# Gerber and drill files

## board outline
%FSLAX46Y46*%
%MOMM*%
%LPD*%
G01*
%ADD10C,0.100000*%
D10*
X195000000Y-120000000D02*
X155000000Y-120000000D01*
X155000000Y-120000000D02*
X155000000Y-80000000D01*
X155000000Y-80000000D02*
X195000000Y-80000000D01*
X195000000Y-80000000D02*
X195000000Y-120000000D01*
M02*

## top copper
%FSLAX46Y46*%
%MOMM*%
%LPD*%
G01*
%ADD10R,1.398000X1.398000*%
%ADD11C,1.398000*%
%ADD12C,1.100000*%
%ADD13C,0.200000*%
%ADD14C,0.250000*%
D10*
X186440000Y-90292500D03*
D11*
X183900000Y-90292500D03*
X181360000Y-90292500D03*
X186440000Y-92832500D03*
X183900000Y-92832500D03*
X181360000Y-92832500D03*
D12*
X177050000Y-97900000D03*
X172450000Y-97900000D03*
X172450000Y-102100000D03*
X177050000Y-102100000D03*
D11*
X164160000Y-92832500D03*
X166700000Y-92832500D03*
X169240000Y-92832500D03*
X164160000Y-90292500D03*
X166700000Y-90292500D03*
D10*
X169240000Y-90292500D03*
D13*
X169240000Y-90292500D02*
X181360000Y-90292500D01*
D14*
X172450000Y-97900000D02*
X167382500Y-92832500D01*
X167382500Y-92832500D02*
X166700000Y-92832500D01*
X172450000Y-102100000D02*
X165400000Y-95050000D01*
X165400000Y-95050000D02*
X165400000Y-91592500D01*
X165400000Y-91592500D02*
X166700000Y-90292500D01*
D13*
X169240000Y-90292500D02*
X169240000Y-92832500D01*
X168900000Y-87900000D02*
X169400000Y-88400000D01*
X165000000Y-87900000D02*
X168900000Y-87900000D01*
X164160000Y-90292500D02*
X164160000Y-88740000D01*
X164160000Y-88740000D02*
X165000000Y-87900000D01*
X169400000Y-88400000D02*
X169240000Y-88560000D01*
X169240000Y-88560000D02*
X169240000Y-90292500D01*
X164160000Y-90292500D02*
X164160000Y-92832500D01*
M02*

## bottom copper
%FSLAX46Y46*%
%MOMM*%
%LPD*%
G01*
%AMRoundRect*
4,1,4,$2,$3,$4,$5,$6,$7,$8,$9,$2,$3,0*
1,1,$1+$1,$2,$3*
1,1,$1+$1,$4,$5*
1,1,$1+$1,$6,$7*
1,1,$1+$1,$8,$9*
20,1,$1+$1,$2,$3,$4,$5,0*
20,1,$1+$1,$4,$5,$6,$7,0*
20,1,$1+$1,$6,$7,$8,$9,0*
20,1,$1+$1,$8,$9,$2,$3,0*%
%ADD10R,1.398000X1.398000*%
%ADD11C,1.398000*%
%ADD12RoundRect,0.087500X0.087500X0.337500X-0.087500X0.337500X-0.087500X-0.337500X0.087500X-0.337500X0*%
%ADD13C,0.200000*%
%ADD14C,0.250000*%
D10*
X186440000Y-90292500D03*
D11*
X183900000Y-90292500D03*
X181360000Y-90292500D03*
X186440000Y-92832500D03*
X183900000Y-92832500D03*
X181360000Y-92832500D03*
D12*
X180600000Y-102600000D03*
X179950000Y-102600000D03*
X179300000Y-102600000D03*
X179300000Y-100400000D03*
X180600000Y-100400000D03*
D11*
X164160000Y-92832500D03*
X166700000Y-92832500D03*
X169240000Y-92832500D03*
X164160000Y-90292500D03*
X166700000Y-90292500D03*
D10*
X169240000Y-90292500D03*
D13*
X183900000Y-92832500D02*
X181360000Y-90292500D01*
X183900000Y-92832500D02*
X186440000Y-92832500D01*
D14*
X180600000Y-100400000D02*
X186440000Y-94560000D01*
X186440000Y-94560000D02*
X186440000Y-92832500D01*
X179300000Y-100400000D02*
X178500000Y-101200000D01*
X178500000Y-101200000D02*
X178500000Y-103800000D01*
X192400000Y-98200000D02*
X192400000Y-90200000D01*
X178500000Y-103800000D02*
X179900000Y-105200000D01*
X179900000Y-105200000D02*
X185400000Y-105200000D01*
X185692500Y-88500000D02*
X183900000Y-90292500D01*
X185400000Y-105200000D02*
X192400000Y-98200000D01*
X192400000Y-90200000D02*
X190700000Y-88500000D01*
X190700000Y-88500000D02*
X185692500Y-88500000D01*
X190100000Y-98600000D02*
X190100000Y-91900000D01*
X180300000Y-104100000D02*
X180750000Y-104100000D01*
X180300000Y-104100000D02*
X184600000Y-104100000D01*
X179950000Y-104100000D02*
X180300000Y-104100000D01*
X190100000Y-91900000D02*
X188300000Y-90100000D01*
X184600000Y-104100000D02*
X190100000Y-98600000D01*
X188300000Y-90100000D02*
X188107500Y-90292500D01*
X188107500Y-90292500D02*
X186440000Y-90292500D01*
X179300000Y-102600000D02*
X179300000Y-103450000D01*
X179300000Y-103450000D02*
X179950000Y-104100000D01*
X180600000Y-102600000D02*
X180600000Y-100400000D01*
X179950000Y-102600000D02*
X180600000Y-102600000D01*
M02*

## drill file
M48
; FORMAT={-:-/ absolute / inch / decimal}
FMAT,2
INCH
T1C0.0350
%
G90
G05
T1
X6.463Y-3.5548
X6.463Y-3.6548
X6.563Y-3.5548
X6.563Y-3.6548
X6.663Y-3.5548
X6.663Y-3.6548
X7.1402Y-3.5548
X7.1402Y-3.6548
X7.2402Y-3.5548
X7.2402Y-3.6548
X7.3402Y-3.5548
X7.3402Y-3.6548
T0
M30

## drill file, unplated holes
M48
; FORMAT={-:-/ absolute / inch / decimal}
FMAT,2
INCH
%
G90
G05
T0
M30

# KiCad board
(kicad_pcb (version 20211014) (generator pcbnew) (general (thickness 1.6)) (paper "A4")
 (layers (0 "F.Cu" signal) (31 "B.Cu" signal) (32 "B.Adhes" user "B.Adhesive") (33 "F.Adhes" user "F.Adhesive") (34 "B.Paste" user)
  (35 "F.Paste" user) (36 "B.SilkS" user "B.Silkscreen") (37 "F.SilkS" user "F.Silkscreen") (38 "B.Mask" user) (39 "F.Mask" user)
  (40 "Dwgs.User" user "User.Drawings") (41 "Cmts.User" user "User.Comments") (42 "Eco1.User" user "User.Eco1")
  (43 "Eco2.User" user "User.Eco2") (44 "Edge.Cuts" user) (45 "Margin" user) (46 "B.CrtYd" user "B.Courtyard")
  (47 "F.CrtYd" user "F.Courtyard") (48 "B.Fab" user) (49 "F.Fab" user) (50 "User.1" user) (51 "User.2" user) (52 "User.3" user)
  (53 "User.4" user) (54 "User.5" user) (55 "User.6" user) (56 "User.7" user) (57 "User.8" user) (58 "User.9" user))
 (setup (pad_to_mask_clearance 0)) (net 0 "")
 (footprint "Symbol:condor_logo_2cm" (layer "F.Cu") (at 165.6 111.2)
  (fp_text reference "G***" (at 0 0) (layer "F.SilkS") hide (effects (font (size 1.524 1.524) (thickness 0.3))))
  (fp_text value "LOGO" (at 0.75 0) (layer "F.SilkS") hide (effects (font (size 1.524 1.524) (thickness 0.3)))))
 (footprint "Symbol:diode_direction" (layer "F.Cu") (at 179.8 100.2 90)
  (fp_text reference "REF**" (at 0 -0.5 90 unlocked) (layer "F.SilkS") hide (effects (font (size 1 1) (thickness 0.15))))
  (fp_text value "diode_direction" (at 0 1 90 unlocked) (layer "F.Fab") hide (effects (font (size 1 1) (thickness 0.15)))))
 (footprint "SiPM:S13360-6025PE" (layer "F.Cu") (at 175 100)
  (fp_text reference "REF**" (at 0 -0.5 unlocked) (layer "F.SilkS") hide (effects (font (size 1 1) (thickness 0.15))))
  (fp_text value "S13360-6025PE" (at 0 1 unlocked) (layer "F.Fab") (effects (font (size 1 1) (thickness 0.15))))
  (pad "1" smd circle (at 2.05 -2.1) (size 1.1 1.1) (layers "F.Cu" "F.Paste" "F.Mask"))
  (pad "2" smd circle (at -2.55 -2.1) (size 1.1 1.1) (layers "F.Cu" "F.Paste" "F.Mask"))
  (pad "3" smd circle (at -2.55 2.1) (size 1.1 1.1) (layers "F.Cu" "F.Paste" "F.Mask"))
  (pad "4" smd circle (at 2.05 2.1) (size 1.1 1.1) (layers "F.Cu" "F.Paste" "F.Mask")))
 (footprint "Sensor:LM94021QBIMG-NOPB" (layer "B.Cu") (at 179.95 101.5 180)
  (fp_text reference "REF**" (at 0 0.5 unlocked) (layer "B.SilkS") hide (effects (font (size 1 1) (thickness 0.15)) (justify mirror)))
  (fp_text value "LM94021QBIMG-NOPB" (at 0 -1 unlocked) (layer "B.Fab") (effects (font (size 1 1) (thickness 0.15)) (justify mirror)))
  (pad "1" smd roundrect (at -0.65 -1.1 180) (size 0.35 0.85) (layers "B.Cu" "B.Paste" "B.Mask") (roundrect_rratio 0.25))
  (pad "2" smd roundrect (at 0 -1.1 180) (size 0.35 0.85) (layers "B.Cu" "B.Paste" "B.Mask") (roundrect_rratio 0.25))
  (pad "3" smd roundrect (at 0.65 -1.1 180) (size 0.35 0.85) (layers "B.Cu" "B.Paste" "B.Mask") (roundrect_rratio 0.25))
  (pad "4" smd roundrect (at 0.65 1.1 180) (size 0.35 0.85) (layers "B.Cu" "B.Paste" "B.Mask") (roundrect_rratio 0.25))
  (pad "5" smd roundrect (at -0.65 1.1 180) (size 0.35 0.85) (layers "B.Cu" "B.Paste" "B.Mask") (roundrect_rratio 0.25)))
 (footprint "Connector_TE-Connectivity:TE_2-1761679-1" (layer "B.Cu") (at 166.7 91.5625 180)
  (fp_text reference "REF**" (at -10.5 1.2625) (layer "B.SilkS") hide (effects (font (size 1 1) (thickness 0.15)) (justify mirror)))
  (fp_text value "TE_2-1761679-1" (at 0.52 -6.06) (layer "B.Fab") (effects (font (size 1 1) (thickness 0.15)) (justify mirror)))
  (pad "1" thru_hole rect locked (at -2.54 1.27 180) (size 1.398 1.398) (drill 0.89) (layers *.Cu *.Mask))
  (pad "2" thru_hole circle locked (at 0 1.27 180) (size 1.398 1.398) (drill 0.89) (layers *.Cu *.Mask))
  (pad "3" thru_hole circle locked (at 2.54 1.27 180) (size 1.398 1.398) (drill 0.89) (layers *.Cu *.Mask))
  (pad "4" thru_hole circle locked (at -2.54 -1.27 180) (size 1.398 1.398) (drill 0.89) (layers *.Cu *.Mask))
  (pad "5" thru_hole circle locked (at 0 -1.27 180) (size 1.398 1.398) (drill 0.89) (layers *.Cu *.Mask))
  (pad "6" thru_hole circle locked (at 2.54 -1.27 180) (size 1.398 1.398) (drill 0.89) (layers *.Cu *.Mask)))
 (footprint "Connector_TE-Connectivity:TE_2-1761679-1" (layer "B.Cu") (at 183.9 91.5625 180)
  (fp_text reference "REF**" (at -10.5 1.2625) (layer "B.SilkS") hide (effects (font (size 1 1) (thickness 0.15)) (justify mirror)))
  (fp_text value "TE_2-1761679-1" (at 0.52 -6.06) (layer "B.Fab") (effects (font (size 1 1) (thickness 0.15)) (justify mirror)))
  (pad "1" thru_hole rect locked (at -2.54 1.27 180) (size 1.398 1.398) (drill 0.89) (layers *.Cu *.Mask))
  (pad "2" thru_hole circle locked (at 0 1.27 180) (size 1.398 1.398) (drill 0.89) (layers *.Cu *.Mask))
  (pad "3" thru_hole circle locked (at 2.54 1.27 180) (size 1.398 1.398) (drill 0.89) (layers *.Cu *.Mask))
  (pad "4" thru_hole circle locked (at -2.54 -1.27 180) (size 1.398 1.398) (drill 0.89) (layers *.Cu *.Mask))
  (pad "5" thru_hole circle locked (at 0 -1.27 180) (size 1.398 1.398) (drill 0.89) (layers *.Cu *.Mask))
  (pad "6" thru_hole circle locked (at 2.54 -1.27 180) (size 1.398 1.398) (drill 0.89) (layers *.Cu *.Mask)))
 (gr_rect (start 195 120) (end 155 80) (layer "Edge.Cuts") (width 0.1) (fill none))
 (segment (start 167.3825 92.8325) (end 166.7 92.8325) (width 0.25) (layer "F.Cu") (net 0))
 (segment (start 164.16 90.2925) (end 164.16 92.8325) (width 0.2) (layer "F.Cu") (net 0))
 (segment (start 172.45 97.9) (end 167.3825 92.8325) (width 0.25) (layer "F.Cu") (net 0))
 (segment (start 169.24 90.2925) (end 169.24 92.8325) (width 0.2) (layer "F.Cu") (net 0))
 (segment (start 164.16 88.74) (end 165 87.9) (width 0.2) (layer "F.Cu") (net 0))
 (segment (start 168.9 87.9) (end 169.4 88.4) (width 0.2) (layer "F.Cu") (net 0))
 (segment (start 165.4 91.5925) (end 166.7 90.2925) (width 0.25) (layer "F.Cu") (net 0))
 (segment (start 164.16 90.2925) (end 164.16 88.74) (width 0.2) (layer "F.Cu") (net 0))
 (segment (start 165.4 95.05) (end 165.4 91.5925) (width 0.25) (layer "F.Cu") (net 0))
 (segment (start 165 87.9) (end 168.9 87.9) (width 0.2) (layer "F.Cu") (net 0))
 (segment (start 172.45 102.1) (end 165.4 95.05) (width 0.25) (layer "F.Cu") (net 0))
 (segment (start 169.24 88.56) (end 169.24 90.2925) (width 0.2) (layer "F.Cu") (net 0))
 (segment (start 169.24 90.2925) (end 181.36 90.2925) (width 0.2) (layer "F.Cu") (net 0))
 (segment (start 169.4 88.4) (end 169.24 88.56) (width 0.2) (layer "F.Cu") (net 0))
 (segment (start 179.9 105.2) (end 185.4 105.2) (width 0.25) (layer "B.Cu") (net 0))
 (segment (start 179.95 104.1) (end 180.3 104.1) (width 0.25) (layer "B.Cu") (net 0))
 (segment (start 192.4 98.2) (end 192.4 90.2) (width 0.25) (layer "B.Cu") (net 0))
 (segment (start 190.1 98.6) (end 190.1 91.9) (width 0.25) (layer "B.Cu") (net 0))
 (segment (start 183.9 92.8325) (end 181.36 90.2925) (width 0.2) (layer "B.Cu") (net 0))
 (segment (start 190.7 88.5) (end 185.6925 88.5) (width 0.25) (layer "B.Cu") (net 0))
 (segment (start 180.6 102.6) (end 180.6 100.4) (width 0.25) (layer "B.Cu") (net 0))
 (segment (start 179.3 100.4) (end 178.5 101.2) (width 0.25) (layer "B.Cu") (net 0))
 (segment (start 185.4 105.2) (end 192.4 98.2) (width 0.25) (layer "B.Cu") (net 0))
 (segment (start 180.3 104.1) (end 180.75 104.1) (width 0.25) (layer "B.Cu") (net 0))
 (segment (start 190.1 91.9) (end 188.3 90.1) (width 0.25) (layer "B.Cu") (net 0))
 (segment (start 178.5 103.8) (end 179.9 105.2) (width 0.25) (layer "B.Cu") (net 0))
 (segment (start 180.6 100.4) (end 186.44 94.56) (width 0.25) (layer "B.Cu") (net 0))
 (segment (start 184.6 104.1) (end 190.1 98.6) (width 0.25) (layer "B.Cu") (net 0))
 (segment (start 185.6925 88.5) (end 183.9 90.2925) (width 0.25) (layer "B.Cu") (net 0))
 (segment (start 186.44 94.56) (end 186.44 92.8325) (width 0.25) (layer "B.Cu") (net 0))
 (segment (start 188.1075 90.2925) (end 186.44 90.2925) (width 0.25) (layer "B.Cu") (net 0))
 (segment (start 178.5 101.2) (end 178.5 103.8) (width 0.25) (layer "B.Cu") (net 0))
 (segment (start 183.9 92.8325) (end 186.44 92.8325) (width 0.2) (layer "B.Cu") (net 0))
 (segment (start 180.3 104.1) (end 184.6 104.1) (width 0.25) (layer "B.Cu") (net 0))
 (segment (start 192.4 90.2) (end 190.7 88.5) (width 0.25) (layer "B.Cu") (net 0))
 (segment (start 179.95 102.6) (end 180.6 102.6) (width 0.25) (layer "B.Cu") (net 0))
 (segment (start 179.3 102.6) (end 179.3 103.45) (width 0.25) (layer "B.Cu") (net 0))
 (segment (start 179.3 103.45) (end 179.95 104.1) (width 0.25) (layer "B.Cu") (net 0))
 (segment (start 188.3 90.1) (end 188.1075 90.2925) (width 0.25) (layer "B.Cu") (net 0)))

